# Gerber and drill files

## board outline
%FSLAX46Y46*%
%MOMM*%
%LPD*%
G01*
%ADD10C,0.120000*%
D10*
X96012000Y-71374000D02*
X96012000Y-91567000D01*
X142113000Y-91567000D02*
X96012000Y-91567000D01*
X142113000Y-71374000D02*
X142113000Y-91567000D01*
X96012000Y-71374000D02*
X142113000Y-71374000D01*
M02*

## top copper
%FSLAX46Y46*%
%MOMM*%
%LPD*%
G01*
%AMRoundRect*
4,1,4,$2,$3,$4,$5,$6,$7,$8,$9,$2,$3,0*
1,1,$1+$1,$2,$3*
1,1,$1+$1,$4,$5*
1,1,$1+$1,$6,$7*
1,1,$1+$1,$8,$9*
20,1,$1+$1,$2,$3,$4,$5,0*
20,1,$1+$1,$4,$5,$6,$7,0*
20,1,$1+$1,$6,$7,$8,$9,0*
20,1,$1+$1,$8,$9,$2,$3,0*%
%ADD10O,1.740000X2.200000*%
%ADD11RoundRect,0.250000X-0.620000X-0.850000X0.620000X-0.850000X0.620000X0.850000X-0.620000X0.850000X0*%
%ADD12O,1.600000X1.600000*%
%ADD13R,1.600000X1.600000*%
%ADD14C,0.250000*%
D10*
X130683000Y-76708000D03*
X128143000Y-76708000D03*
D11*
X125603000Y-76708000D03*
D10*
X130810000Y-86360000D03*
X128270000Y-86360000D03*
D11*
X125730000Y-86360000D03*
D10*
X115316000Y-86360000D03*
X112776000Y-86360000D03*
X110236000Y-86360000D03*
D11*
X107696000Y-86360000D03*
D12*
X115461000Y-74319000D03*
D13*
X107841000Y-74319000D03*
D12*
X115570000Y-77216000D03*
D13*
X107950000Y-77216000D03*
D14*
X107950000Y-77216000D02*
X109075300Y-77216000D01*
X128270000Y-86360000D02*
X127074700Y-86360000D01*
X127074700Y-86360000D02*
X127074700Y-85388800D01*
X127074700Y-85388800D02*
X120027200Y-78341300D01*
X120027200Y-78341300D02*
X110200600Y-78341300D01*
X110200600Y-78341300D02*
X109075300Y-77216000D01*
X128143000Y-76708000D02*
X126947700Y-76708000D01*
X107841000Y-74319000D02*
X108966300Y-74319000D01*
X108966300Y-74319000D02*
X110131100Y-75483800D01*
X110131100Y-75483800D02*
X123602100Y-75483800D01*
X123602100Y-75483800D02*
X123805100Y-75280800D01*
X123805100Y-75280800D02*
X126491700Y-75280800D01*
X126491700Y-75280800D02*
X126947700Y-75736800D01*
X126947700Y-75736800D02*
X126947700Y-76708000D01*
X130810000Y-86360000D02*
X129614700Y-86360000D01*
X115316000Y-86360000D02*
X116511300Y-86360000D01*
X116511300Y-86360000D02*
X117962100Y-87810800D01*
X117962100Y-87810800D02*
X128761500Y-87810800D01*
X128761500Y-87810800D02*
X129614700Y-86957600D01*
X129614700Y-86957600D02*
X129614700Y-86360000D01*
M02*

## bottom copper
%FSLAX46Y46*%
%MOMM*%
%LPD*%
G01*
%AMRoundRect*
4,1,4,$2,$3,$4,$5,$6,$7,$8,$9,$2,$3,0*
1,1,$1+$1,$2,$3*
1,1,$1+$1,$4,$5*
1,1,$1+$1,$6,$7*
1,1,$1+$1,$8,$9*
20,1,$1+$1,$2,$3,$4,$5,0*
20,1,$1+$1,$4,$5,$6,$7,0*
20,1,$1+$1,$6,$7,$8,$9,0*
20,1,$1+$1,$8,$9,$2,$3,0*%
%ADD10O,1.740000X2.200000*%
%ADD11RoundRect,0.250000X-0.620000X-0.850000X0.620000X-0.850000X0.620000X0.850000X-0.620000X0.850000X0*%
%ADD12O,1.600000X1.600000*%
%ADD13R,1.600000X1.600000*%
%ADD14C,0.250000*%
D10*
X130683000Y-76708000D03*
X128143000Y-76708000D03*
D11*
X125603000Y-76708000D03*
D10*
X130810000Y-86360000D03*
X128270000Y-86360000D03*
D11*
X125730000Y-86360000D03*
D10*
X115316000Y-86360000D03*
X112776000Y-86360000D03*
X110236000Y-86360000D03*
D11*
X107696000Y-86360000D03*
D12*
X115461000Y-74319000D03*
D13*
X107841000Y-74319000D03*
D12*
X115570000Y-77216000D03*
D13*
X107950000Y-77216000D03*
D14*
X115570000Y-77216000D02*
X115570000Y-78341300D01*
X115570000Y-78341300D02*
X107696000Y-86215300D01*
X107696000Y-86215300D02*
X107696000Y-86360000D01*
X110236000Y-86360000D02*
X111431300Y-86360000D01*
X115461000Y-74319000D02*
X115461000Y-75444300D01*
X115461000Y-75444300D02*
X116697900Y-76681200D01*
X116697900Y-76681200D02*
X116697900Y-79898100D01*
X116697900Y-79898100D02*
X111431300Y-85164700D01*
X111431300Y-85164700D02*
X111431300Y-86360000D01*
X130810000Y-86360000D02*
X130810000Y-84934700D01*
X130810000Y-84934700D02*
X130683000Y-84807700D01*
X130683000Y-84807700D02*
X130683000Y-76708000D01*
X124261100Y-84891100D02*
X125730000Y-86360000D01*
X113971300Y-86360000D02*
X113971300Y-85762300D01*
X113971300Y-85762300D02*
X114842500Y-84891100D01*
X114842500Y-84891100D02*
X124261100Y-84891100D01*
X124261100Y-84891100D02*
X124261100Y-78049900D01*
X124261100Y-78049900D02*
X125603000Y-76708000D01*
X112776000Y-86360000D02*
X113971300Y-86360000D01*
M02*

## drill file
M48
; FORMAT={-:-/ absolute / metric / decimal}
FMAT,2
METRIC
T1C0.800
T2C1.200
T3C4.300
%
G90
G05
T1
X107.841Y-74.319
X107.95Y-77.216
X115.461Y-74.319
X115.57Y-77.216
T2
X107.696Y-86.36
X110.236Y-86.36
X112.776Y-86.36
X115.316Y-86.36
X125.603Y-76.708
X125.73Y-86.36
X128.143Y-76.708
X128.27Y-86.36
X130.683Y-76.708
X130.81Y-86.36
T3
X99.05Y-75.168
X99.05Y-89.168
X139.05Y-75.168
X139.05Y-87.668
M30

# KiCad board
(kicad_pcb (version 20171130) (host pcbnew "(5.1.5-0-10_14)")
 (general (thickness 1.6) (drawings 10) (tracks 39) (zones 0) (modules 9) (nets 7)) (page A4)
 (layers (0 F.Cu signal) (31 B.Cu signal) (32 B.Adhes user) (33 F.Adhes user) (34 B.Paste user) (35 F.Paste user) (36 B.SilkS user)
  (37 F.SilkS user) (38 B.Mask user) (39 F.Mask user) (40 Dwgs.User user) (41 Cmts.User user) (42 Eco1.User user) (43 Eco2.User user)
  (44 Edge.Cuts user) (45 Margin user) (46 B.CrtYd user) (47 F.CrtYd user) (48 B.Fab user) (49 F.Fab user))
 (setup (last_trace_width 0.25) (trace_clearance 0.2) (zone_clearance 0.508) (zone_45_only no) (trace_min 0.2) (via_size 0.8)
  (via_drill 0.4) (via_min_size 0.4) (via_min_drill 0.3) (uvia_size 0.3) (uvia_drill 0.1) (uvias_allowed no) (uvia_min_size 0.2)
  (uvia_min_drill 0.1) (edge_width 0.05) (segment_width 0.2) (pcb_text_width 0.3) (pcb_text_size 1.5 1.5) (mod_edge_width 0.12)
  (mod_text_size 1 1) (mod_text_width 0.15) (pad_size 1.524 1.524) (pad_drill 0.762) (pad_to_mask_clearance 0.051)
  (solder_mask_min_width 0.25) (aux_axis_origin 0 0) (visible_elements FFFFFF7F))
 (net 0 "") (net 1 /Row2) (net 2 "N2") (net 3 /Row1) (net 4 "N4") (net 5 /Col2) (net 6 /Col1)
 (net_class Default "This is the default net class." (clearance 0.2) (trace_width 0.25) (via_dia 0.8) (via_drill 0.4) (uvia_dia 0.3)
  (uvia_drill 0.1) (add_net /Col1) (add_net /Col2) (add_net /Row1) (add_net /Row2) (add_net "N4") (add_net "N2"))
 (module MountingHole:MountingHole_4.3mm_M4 (layer F.Cu) (at 99.05 75.168)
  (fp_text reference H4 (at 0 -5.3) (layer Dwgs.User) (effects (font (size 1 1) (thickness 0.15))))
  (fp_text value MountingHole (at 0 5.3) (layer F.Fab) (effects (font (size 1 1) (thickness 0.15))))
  (pad 1 np_thru_hole circle (at 0 0) (size 4.3 4.3) (drill 4.3) (layers *.Cu *.Mask)))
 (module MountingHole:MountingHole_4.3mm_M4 (layer F.Cu) (at 99.05 89.168)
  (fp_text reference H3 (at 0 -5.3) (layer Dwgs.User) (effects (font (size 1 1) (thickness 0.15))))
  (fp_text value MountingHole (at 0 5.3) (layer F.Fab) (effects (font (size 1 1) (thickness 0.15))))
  (pad 1 np_thru_hole circle (at 0 0) (size 4.3 4.3) (drill 4.3) (layers *.Cu *.Mask)))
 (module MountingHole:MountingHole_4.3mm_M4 (layer F.Cu) (at 139.05 87.668)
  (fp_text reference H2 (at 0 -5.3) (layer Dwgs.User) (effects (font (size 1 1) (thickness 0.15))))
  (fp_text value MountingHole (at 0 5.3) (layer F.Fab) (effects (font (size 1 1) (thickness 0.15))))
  (pad 1 np_thru_hole circle (at 0 0) (size 4.3 4.3) (drill 4.3) (layers *.Cu *.Mask)))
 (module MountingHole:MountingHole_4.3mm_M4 (layer F.Cu) (at 139.05 75.168)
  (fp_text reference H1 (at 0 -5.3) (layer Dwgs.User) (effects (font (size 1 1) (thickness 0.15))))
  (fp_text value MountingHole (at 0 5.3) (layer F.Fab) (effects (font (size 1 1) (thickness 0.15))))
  (pad 1 np_thru_hole circle (at 0 0) (size 4.3 4.3) (drill 4.3) (layers *.Cu *.Mask)))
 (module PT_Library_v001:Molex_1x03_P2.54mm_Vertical (layer F.Cu) (at 125.603 76.708)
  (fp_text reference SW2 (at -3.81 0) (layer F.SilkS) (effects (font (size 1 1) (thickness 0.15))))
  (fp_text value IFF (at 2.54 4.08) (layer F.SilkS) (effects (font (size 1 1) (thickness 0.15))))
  (pad 3 thru_hole oval (at 5.08 0) (size 1.74 2.2) (drill 1.2) (layers *.Cu *.Mask) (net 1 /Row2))
  (pad 2 thru_hole oval (at 2.54 0) (size 1.74 2.2) (drill 1.2) (layers *.Cu *.Mask) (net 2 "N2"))
  (pad 1 thru_hole roundrect (at 0 0) (size 1.74 2.2) (drill 1.2) (layers *.Cu *.Mask) (roundrect_rratio 0.143678) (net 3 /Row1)))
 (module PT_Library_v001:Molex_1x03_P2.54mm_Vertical (layer F.Cu) (at 125.73 86.36)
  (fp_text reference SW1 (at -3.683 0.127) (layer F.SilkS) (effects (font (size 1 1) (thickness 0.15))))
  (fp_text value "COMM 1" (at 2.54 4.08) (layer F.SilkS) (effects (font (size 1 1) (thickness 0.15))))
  (pad 3 thru_hole oval (at 5.08 0) (size 1.74 2.2) (drill 1.2) (layers *.Cu *.Mask) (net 1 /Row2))
  (pad 2 thru_hole oval (at 2.54 0) (size 1.74 2.2) (drill 1.2) (layers *.Cu *.Mask) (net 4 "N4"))
  (pad 1 thru_hole roundrect (at 0 0) (size 1.74 2.2) (drill 1.2) (layers *.Cu *.Mask) (roundrect_rratio 0.143678) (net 3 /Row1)))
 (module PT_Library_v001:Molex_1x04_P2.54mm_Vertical (layer F.Cu) (at 107.696 86.36)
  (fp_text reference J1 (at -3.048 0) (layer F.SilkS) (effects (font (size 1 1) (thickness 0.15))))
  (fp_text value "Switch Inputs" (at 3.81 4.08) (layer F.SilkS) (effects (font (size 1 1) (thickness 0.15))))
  (pad 4 thru_hole oval (at 7.62 0) (size 1.74 2.2) (drill 1.2) (layers *.Cu *.Mask) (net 1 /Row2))
  (pad 3 thru_hole oval (at 5.08 0) (size 1.74 2.2) (drill 1.2) (layers *.Cu *.Mask) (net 3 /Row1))
  (pad 2 thru_hole oval (at 2.54 0) (size 1.74 2.2) (drill 1.2) (layers *.Cu *.Mask) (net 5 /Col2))
  (pad 1 thru_hole roundrect (at 0 0) (size 1.74 2.2) (drill 1.2) (layers *.Cu *.Mask) (roundrect_rratio 0.143678) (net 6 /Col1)))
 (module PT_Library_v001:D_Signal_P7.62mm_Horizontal (layer F.Cu) (at 107.841 74.319)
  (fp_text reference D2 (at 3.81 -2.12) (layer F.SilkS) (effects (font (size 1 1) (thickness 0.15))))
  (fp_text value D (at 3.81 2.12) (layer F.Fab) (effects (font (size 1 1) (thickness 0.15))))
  (pad 2 thru_hole oval (at 7.62 0) (size 1.6 1.6) (drill 0.8) (layers *.Cu *.Mask) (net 5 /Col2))
  (pad 1 thru_hole rect (at 0 0) (size 1.6 1.6) (drill 0.8) (layers *.Cu *.Mask) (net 2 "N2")))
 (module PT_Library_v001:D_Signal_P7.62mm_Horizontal (layer F.Cu) (at 107.95 77.216)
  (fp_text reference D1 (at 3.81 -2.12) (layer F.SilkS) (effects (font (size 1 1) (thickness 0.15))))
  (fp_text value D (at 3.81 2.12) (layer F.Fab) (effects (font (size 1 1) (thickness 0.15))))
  (pad 2 thru_hole oval (at 7.62 0) (size 1.6 1.6) (drill 0.8) (layers *.Cu *.Mask) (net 6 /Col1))
  (pad 1 thru_hole rect (at 0 0) (size 1.6 1.6) (drill 0.8) (layers *.Cu *.Mask) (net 4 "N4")))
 (gr_line (start 96.012 71.374) (end 96.012 91.567) (layer Edge.Cuts) (width 0.12))
 (gr_line (start 142.113 91.567) (end 96.012 91.567) (layer Edge.Cuts) (width 0.12))
 (gr_line (start 142.113 71.374) (end 142.113 91.567) (layer Edge.Cuts) (width 0.12))
 (gr_line (start 96.012 71.374) (end 142.113 71.374) (layer Edge.Cuts) (width 0.12))
 (segment (start 115.57 77.216) (end 115.57 78.3413) (width 0.25) (layer B.Cu) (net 6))
 (segment (start 115.57 78.3413) (end 107.696 86.2153) (width 0.25) (layer B.Cu) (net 6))
 (segment (start 107.696 86.2153) (end 107.696 86.36) (width 0.25) (layer B.Cu) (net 6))
 (segment (start 107.95 77.216) (end 109.0753 77.216) (width 0.25) (layer F.Cu) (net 4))
 (segment (start 128.27 86.36) (end 127.0747 86.36) (width 0.25) (layer F.Cu) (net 4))
 (segment (start 127.0747 86.36) (end 127.0747 85.3888) (width 0.25) (layer F.Cu) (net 4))
 (segment (start 127.0747 85.3888) (end 120.0272 78.3413) (width 0.25) (layer F.Cu) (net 4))
 (segment (start 120.0272 78.3413) (end 110.2006 78.3413) (width 0.25) (layer F.Cu) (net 4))
 (segment (start 110.2006 78.3413) (end 109.0753 77.216) (width 0.25) (layer F.Cu) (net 4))
 (segment (start 110.236 86.36) (end 111.4313 86.36) (width 0.25) (layer B.Cu) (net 5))
 (segment (start 115.461 74.319) (end 115.461 75.4443) (width 0.25) (layer B.Cu) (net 5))
 (segment (start 115.461 75.4443) (end 116.6979 76.6812) (width 0.25) (layer B.Cu) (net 5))
 (segment (start 116.6979 76.6812) (end 116.6979 79.8981) (width 0.25) (layer B.Cu) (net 5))
 (segment (start 116.6979 79.8981) (end 111.4313 85.1647) (width 0.25) (layer B.Cu) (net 5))
 (segment (start 111.4313 85.1647) (end 111.4313 86.36) (width 0.25) (layer B.Cu) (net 5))
 (segment (start 128.143 76.708) (end 126.9477 76.708) (width 0.25) (layer F.Cu) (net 2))
 (segment (start 107.841 74.319) (end 108.9663 74.319) (width 0.25) (layer F.Cu) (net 2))
 (segment (start 108.9663 74.319) (end 110.1311 75.4838) (width 0.25) (layer F.Cu) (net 2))
 (segment (start 110.1311 75.4838) (end 123.6021 75.4838) (width 0.25) (layer F.Cu) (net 2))
 (segment (start 123.6021 75.4838) (end 123.8051 75.2808) (width 0.25) (layer F.Cu) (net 2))
 (segment (start 123.8051 75.2808) (end 126.4917 75.2808) (width 0.25) (layer F.Cu) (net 2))
 (segment (start 126.4917 75.2808) (end 126.9477 75.7368) (width 0.25) (layer F.Cu) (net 2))
 (segment (start 126.9477 75.7368) (end 126.9477 76.708) (width 0.25) (layer F.Cu) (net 2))
 (segment (start 130.81 86.36) (end 130.81 84.9347) (width 0.25) (layer B.Cu) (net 1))
 (segment (start 130.81 84.9347) (end 130.683 84.8077) (width 0.25) (layer B.Cu) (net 1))
 (segment (start 130.683 84.8077) (end 130.683 76.708) (width 0.25) (layer B.Cu) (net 1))
 (segment (start 130.81 86.36) (end 129.6147 86.36) (width 0.25) (layer F.Cu) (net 1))
 (segment (start 115.316 86.36) (end 116.5113 86.36) (width 0.25) (layer F.Cu) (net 1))
 (segment (start 116.5113 86.36) (end 117.9621 87.8108) (width 0.25) (layer F.Cu) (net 1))
 (segment (start 117.9621 87.8108) (end 128.7615 87.8108) (width 0.25) (layer F.Cu) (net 1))
 (segment (start 128.7615 87.8108) (end 129.6147 86.9576) (width 0.25) (layer F.Cu) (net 1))
 (segment (start 129.6147 86.9576) (end 129.6147 86.36) (width 0.25) (layer F.Cu) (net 1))
 (segment (start 124.2611 84.8911) (end 125.73 86.36) (width 0.25) (layer B.Cu) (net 3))
 (segment (start 113.9713 86.36) (end 113.9713 85.7623) (width 0.25) (layer B.Cu) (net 3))
 (segment (start 113.9713 85.7623) (end 114.8425 84.8911) (width 0.25) (layer B.Cu) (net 3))
 (segment (start 114.8425 84.8911) (end 124.2611 84.8911) (width 0.25) (layer B.Cu) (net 3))
 (segment (start 124.2611 84.8911) (end 124.2611 78.0499) (width 0.25) (layer B.Cu) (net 3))
 (segment (start 124.2611 78.0499) (end 125.603 76.708) (width 0.25) (layer B.Cu) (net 3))
 (segment (start 112.776 86.36) (end 113.9713 86.36) (width 0.25) (layer B.Cu) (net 3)))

